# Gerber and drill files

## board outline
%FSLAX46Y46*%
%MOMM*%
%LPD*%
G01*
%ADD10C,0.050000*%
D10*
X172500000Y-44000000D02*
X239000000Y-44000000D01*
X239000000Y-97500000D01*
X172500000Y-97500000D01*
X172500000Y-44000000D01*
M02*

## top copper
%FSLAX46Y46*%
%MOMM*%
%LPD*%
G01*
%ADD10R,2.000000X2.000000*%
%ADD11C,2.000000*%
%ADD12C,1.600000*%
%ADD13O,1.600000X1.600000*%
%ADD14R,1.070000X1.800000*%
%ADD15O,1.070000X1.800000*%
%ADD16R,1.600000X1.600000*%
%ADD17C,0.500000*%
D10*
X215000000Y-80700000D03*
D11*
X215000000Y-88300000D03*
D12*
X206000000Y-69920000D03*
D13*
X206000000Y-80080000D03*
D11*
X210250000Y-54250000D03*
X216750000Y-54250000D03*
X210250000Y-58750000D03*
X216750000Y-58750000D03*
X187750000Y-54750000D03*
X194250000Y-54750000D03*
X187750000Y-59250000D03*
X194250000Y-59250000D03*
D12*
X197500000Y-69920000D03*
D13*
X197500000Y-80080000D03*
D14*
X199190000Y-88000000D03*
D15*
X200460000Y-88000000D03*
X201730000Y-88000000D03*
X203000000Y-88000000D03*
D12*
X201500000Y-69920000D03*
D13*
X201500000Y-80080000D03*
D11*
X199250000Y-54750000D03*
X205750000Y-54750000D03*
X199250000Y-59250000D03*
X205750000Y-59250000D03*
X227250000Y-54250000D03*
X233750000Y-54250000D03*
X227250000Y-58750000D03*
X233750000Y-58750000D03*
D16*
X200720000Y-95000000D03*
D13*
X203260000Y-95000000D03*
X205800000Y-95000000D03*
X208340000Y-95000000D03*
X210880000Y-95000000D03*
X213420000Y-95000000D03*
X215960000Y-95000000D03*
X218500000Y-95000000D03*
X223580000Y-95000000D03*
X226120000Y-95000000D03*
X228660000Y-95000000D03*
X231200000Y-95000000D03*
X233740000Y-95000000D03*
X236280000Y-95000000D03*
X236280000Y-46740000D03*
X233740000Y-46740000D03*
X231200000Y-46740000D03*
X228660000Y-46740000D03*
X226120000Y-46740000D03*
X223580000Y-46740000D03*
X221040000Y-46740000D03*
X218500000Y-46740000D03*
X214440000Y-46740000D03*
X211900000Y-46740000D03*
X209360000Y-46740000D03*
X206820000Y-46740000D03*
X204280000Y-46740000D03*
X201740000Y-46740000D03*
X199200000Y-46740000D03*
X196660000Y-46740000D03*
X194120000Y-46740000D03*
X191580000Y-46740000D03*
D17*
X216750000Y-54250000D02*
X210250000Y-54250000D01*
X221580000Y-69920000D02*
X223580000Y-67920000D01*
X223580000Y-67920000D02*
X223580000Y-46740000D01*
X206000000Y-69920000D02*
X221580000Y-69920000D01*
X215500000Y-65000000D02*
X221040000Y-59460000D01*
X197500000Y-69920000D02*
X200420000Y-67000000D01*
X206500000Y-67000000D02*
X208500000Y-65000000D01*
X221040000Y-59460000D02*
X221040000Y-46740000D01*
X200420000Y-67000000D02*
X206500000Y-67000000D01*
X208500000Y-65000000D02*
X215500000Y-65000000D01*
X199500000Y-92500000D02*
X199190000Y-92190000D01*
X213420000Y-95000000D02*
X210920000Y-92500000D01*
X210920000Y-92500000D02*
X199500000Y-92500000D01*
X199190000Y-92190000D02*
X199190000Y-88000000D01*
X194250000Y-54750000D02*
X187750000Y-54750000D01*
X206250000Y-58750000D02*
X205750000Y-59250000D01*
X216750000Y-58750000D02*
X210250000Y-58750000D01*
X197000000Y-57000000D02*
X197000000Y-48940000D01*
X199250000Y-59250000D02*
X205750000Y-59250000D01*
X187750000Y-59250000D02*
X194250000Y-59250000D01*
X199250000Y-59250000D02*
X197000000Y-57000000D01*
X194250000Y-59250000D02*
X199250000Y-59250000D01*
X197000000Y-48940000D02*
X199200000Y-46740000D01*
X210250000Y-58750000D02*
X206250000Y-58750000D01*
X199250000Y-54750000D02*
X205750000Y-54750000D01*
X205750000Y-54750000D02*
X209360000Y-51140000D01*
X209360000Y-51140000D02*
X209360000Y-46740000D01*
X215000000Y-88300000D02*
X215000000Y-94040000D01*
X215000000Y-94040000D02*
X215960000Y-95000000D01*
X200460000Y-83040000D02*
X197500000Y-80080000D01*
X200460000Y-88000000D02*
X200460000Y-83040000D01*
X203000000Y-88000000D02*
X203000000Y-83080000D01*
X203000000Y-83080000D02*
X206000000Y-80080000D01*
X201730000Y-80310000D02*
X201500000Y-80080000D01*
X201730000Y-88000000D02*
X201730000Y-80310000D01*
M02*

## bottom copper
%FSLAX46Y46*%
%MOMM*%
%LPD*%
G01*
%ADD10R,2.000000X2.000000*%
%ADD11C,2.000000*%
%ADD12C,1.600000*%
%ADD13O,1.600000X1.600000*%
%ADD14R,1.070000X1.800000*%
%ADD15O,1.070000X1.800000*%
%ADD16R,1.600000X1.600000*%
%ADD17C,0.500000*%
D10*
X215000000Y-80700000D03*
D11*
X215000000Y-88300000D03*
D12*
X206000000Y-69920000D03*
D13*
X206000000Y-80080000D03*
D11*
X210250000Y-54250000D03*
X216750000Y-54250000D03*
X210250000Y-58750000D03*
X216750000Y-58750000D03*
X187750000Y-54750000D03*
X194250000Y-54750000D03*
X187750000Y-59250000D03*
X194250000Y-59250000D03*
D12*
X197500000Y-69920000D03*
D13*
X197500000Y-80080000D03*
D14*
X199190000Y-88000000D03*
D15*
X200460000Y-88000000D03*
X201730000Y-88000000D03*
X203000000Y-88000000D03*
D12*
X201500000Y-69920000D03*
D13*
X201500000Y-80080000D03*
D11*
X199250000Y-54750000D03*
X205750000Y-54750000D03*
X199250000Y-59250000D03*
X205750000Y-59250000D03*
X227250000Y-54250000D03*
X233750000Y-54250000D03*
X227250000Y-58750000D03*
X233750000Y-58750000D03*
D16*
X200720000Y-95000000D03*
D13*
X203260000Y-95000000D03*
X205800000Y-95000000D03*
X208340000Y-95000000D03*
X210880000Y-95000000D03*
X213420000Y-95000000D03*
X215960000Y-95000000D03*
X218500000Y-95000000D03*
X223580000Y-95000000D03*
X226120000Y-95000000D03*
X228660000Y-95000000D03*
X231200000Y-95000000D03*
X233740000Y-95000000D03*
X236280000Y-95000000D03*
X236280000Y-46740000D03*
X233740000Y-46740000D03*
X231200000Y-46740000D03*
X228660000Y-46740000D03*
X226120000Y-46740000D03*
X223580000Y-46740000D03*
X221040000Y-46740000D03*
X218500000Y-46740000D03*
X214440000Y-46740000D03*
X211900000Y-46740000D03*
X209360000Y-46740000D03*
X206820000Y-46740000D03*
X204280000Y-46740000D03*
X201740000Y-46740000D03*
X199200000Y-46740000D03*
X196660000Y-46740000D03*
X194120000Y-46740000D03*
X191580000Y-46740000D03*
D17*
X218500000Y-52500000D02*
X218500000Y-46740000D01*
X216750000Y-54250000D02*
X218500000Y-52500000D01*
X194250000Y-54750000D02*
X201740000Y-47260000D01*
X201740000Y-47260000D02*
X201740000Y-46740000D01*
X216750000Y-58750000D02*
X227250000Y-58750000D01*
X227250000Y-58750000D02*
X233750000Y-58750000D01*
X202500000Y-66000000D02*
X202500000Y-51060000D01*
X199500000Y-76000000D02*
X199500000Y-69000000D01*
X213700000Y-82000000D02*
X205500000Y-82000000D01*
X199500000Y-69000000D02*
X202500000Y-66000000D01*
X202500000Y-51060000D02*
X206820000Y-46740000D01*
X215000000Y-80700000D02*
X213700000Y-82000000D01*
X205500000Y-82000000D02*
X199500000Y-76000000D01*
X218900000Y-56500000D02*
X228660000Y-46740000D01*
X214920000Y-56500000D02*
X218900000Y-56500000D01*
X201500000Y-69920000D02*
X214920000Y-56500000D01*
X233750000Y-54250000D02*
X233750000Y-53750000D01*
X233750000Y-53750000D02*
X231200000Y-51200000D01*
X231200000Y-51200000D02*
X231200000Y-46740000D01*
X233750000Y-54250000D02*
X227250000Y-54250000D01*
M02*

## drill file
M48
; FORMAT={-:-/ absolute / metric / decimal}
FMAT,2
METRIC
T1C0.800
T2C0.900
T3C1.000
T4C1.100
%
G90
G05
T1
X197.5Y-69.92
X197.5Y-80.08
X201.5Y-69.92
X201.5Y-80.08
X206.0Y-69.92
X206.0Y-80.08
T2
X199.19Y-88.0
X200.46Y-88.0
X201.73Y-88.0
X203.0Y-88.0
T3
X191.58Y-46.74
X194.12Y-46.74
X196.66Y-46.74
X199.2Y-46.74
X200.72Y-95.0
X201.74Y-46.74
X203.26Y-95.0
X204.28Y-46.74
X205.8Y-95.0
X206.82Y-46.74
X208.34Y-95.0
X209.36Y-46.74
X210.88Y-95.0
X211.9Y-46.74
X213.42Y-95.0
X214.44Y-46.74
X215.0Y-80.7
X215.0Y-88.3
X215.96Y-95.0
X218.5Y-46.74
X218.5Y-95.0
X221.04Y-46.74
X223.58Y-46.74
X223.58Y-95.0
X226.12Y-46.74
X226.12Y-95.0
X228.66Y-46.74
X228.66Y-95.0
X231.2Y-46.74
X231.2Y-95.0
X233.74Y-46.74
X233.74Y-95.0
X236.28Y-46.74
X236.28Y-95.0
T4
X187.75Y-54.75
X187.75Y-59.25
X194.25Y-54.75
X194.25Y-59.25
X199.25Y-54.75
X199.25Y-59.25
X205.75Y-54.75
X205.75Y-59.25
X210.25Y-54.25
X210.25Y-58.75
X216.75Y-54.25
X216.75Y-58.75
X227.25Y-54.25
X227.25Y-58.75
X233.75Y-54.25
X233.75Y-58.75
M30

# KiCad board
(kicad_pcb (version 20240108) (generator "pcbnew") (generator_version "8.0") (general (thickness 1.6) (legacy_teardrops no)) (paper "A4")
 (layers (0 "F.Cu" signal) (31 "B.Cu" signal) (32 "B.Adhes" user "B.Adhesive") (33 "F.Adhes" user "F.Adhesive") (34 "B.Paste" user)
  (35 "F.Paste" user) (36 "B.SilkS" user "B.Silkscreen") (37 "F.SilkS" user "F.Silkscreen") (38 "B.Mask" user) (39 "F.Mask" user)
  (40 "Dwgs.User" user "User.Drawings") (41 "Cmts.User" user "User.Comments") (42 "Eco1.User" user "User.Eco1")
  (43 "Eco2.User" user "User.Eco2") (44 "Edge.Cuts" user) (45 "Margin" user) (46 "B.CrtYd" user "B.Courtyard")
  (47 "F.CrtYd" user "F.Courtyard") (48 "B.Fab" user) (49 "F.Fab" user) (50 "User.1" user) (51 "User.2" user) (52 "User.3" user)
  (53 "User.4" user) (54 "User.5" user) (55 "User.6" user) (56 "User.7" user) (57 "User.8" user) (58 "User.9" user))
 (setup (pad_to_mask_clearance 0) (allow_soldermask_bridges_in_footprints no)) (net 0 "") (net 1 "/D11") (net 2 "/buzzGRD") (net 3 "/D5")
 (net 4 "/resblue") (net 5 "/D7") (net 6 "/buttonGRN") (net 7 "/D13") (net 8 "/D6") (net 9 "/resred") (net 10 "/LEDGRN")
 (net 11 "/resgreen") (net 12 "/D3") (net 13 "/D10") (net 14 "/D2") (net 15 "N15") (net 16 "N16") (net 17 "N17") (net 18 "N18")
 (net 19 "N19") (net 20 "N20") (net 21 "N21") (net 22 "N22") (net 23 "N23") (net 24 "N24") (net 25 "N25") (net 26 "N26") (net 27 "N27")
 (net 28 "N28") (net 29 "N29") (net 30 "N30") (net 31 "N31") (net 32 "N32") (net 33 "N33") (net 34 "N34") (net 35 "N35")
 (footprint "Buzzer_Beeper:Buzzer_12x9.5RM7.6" (layer "F.Cu") (at 215 80.7 -90)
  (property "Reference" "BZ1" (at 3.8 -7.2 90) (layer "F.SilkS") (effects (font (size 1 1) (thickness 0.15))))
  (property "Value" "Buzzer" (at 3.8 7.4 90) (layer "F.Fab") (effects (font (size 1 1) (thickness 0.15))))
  (pad "1" thru_hole rect (at 0 0 270) (size 2 2) (drill 1) (layers "*.Cu" "*.Mask") (remove_unused_layers no) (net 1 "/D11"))
  (pad "2" thru_hole circle (at 7.6 0 270) (size 2 2) (drill 1) (layers "*.Cu" "*.Mask") (remove_unused_layers no) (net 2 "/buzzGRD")))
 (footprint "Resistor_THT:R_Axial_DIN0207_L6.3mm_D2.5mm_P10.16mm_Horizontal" (layer "F.Cu") (at 206 69.92 -90)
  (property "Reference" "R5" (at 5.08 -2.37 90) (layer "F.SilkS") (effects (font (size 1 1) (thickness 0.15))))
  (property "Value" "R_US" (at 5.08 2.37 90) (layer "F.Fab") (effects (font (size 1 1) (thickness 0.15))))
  (pad "1" thru_hole circle (at 0 0 270) (size 1.6 1.6) (drill 0.8) (layers "*.Cu" "*.Mask") (remove_unused_layers no) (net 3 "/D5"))
  (pad "2" thru_hole oval (at 10.16 0 270) (size 1.6 1.6) (drill 0.8) (layers "*.Cu" "*.Mask") (remove_unused_layers no) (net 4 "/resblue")))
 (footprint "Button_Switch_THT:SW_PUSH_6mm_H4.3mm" (layer "F.Cu") (at 210.25 54.25)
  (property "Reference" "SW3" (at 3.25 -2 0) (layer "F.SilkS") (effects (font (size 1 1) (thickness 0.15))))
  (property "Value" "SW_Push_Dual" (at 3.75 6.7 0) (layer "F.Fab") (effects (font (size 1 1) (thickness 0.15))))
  (pad "1" thru_hole circle (at 0 0 90) (size 2 2) (drill 1.1) (layers "*.Cu" "*.Mask") (remove_unused_layers no) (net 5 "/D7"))
  (pad "1" thru_hole circle (at 6.5 0 90) (size 2 2) (drill 1.1) (layers "*.Cu" "*.Mask") (remove_unused_layers no) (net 5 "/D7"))
  (pad "2" thru_hole circle (at 0 4.5 90) (size 2 2) (drill 1.1) (layers "*.Cu" "*.Mask") (remove_unused_layers no) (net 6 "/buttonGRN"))
  (pad "2" thru_hole circle (at 6.5 4.5 90) (size 2 2) (drill 1.1) (layers "*.Cu" "*.Mask") (remove_unused_layers no) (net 6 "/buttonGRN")))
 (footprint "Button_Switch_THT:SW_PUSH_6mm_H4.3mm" (layer "F.Cu") (at 187.75 54.75)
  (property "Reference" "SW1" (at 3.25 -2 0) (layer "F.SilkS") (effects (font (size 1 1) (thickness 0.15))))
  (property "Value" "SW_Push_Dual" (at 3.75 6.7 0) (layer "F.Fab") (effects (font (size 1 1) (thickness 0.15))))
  (pad "1" thru_hole circle (at 0 0 90) (size 2 2) (drill 1.1) (layers "*.Cu" "*.Mask") (remove_unused_layers no) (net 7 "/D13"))
  (pad "1" thru_hole circle (at 6.5 0 90) (size 2 2) (drill 1.1) (layers "*.Cu" "*.Mask") (remove_unused_layers no) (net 7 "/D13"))
  (pad "2" thru_hole circle (at 0 4.5 90) (size 2 2) (drill 1.1) (layers "*.Cu" "*.Mask") (remove_unused_layers no) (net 6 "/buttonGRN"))
  (pad "2" thru_hole circle (at 6.5 4.5 90) (size 2 2) (drill 1.1) (layers "*.Cu" "*.Mask") (remove_unused_layers no) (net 6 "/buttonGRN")))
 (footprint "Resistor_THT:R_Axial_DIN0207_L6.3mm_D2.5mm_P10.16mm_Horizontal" (layer "F.Cu") (at 197.5 69.92 -90)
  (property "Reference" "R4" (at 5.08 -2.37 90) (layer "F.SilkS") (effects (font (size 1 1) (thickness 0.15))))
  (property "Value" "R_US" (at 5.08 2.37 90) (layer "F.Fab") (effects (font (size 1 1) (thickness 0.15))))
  (pad "1" thru_hole circle (at 0 0 270) (size 1.6 1.6) (drill 0.8) (layers "*.Cu" "*.Mask") (remove_unused_layers no) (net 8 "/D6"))
  (pad "2" thru_hole oval (at 10.16 0 270) (size 1.6 1.6) (drill 0.8) (layers "*.Cu" "*.Mask") (remove_unused_layers no) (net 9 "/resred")))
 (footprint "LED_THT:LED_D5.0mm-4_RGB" (layer "F.Cu") (at 199.19 88)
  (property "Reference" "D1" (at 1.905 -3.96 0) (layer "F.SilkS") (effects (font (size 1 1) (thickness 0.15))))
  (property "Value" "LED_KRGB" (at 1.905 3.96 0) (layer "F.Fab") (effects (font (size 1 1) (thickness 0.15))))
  (pad "1" thru_hole rect (at 0 0) (size 1.07 1.8) (drill 0.9) (layers "*.Cu" "*.Mask") (remove_unused_layers no) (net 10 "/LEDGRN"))
  (pad "2" thru_hole oval (at 1.27 0) (size 1.07 1.8) (drill 0.9) (layers "*.Cu" "*.Mask") (remove_unused_layers no) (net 9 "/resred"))
  (pad "3" thru_hole oval (at 2.54 0) (size 1.07 1.8) (drill 0.9) (layers "*.Cu" "*.Mask") (remove_unused_layers no) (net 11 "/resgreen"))
  (pad "4" thru_hole oval (at 3.81 0) (size 1.07 1.8) (drill 0.9) (layers "*.Cu" "*.Mask") (remove_unused_layers no) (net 4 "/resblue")))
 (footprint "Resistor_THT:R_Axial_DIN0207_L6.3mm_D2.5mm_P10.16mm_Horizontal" (layer "F.Cu") (at 201.5 69.92 -90)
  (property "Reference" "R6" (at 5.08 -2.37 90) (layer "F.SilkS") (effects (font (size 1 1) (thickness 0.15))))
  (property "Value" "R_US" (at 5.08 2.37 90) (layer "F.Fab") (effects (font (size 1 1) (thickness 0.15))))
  (pad "1" thru_hole circle (at 0 0 270) (size 1.6 1.6) (drill 0.8) (layers "*.Cu" "*.Mask") (remove_unused_layers no) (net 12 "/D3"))
  (pad "2" thru_hole oval (at 10.16 0 270) (size 1.6 1.6) (drill 0.8) (layers "*.Cu" "*.Mask") (remove_unused_layers no)
   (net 11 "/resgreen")))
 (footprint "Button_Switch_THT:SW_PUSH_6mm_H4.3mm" (layer "F.Cu") (at 199.25 54.75)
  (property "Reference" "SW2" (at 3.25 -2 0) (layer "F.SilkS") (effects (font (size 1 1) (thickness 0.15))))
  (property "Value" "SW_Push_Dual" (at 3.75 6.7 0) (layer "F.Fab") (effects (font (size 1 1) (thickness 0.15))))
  (pad "1" thru_hole circle (at 0 0 90) (size 2 2) (drill 1.1) (layers "*.Cu" "*.Mask") (remove_unused_layers no) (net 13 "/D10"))
  (pad "1" thru_hole circle (at 6.5 0 90) (size 2 2) (drill 1.1) (layers "*.Cu" "*.Mask") (remove_unused_layers no) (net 13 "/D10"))
  (pad "2" thru_hole circle (at 0 4.5 90) (size 2 2) (drill 1.1) (layers "*.Cu" "*.Mask") (remove_unused_layers no) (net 6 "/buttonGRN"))
  (pad "2" thru_hole circle (at 6.5 4.5 90) (size 2 2) (drill 1.1) (layers "*.Cu" "*.Mask") (remove_unused_layers no) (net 6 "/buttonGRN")))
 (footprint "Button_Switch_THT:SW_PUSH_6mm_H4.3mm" (layer "F.Cu") (at 227.25 54.25)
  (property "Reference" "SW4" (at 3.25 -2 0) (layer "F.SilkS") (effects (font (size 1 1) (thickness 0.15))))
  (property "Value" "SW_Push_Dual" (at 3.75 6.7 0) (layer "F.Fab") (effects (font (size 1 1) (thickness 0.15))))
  (pad "1" thru_hole circle (at 0 0 90) (size 2 2) (drill 1.1) (layers "*.Cu" "*.Mask") (remove_unused_layers no) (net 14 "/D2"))
  (pad "1" thru_hole circle (at 6.5 0 90) (size 2 2) (drill 1.1) (layers "*.Cu" "*.Mask") (remove_unused_layers no) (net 14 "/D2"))
  (pad "2" thru_hole circle (at 0 4.5 90) (size 2 2) (drill 1.1) (layers "*.Cu" "*.Mask") (remove_unused_layers no) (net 6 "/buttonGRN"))
  (pad "2" thru_hole circle (at 6.5 4.5 90) (size 2 2) (drill 1.1) (layers "*.Cu" "*.Mask") (remove_unused_layers no) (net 6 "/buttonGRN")))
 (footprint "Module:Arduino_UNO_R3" (layer "B.Cu") (at 200.72 95)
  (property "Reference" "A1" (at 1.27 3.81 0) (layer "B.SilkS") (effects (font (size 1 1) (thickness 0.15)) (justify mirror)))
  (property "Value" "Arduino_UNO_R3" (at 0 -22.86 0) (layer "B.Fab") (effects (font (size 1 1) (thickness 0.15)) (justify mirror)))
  (pad "1" thru_hole rect (at 0 0 270) (size 1.6 1.6) (drill 1) (layers "*.Cu" "*.Mask") (remove_unused_layers no) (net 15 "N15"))
  (pad "2" thru_hole oval (at 2.54 0 270) (size 1.6 1.6) (drill 1) (layers "*.Cu" "*.Mask") (remove_unused_layers no) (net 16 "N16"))
  (pad "3" thru_hole oval (at 5.08 0 270) (size 1.6 1.6) (drill 1) (layers "*.Cu" "*.Mask") (remove_unused_layers no) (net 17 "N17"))
  (pad "4" thru_hole oval (at 7.62 0 270) (size 1.6 1.6) (drill 1) (layers "*.Cu" "*.Mask") (remove_unused_layers no) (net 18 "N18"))
  (pad "5" thru_hole oval (at 10.16 0 270) (size 1.6 1.6) (drill 1) (layers "*.Cu" "*.Mask") (remove_unused_layers no) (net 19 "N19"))
  (pad "6" thru_hole oval (at 12.7 0 270) (size 1.6 1.6) (drill 1) (layers "*.Cu" "*.Mask") (remove_unused_layers no) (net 10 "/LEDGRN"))
  (pad "7" thru_hole oval (at 15.24 0 270) (size 1.6 1.6) (drill 1) (layers "*.Cu" "*.Mask") (remove_unused_layers no) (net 2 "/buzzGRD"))
  (pad "8" thru_hole oval (at 17.78 0 270) (size 1.6 1.6) (drill 1) (layers "*.Cu" "*.Mask") (remove_unused_layers no) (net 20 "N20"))
  (pad "9" thru_hole oval (at 22.86 0 270) (size 1.6 1.6) (drill 1) (layers "*.Cu" "*.Mask") (remove_unused_layers no) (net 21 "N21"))
  (pad "10" thru_hole oval (at 25.4 0 270) (size 1.6 1.6) (drill 1) (layers "*.Cu" "*.Mask") (remove_unused_layers no) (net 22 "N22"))
  (pad "11" thru_hole oval (at 27.94 0 270) (size 1.6 1.6) (drill 1) (layers "*.Cu" "*.Mask") (remove_unused_layers no) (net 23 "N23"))
  (pad "12" thru_hole oval (at 30.48 0 270) (size 1.6 1.6) (drill 1) (layers "*.Cu" "*.Mask") (remove_unused_layers no) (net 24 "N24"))
  (pad "13" thru_hole oval (at 33.02 0 270) (size 1.6 1.6) (drill 1) (layers "*.Cu" "*.Mask") (remove_unused_layers no) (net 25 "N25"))
  (pad "14" thru_hole oval (at 35.56 0 270) (size 1.6 1.6) (drill 1) (layers "*.Cu" "*.Mask") (remove_unused_layers no) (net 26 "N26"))
  (pad "15" thru_hole oval (at 35.56 -48.26 270) (size 1.6 1.6) (drill 1) (layers "*.Cu" "*.Mask") (remove_unused_layers no) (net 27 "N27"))
  (pad "16" thru_hole oval (at 33.02 -48.26 270) (size 1.6 1.6) (drill 1) (layers "*.Cu" "*.Mask") (remove_unused_layers no) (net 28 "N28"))
  (pad "17" thru_hole oval (at 30.48 -48.26 270) (size 1.6 1.6) (drill 1) (layers "*.Cu" "*.Mask") (remove_unused_layers no) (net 14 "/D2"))
  (pad "18" thru_hole oval (at 27.94 -48.26 270) (size 1.6 1.6) (drill 1) (layers "*.Cu" "*.Mask") (remove_unused_layers no) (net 12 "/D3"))
  (pad "19" thru_hole oval (at 25.4 -48.26 270) (size 1.6 1.6) (drill 1) (layers "*.Cu" "*.Mask") (remove_unused_layers no) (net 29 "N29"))
  (pad "20" thru_hole oval (at 22.86 -48.26 270) (size 1.6 1.6) (drill 1) (layers "*.Cu" "*.Mask") (remove_unused_layers no) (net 3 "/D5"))
  (pad "21" thru_hole oval (at 20.32 -48.26 270) (size 1.6 1.6) (drill 1) (layers "*.Cu" "*.Mask") (remove_unused_layers no) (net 8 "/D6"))
  (pad "22" thru_hole oval (at 17.78 -48.26 270) (size 1.6 1.6) (drill 1) (layers "*.Cu" "*.Mask") (remove_unused_layers no) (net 5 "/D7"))
  (pad "23" thru_hole oval (at 13.72 -48.26 270) (size 1.6 1.6) (drill 1) (layers "*.Cu" "*.Mask") (remove_unused_layers no) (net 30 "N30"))
  (pad "24" thru_hole oval (at 11.18 -48.26 270) (size 1.6 1.6) (drill 1) (layers "*.Cu" "*.Mask") (remove_unused_layers no) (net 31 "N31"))
  (pad "25" thru_hole oval (at 8.64 -48.26 270) (size 1.6 1.6) (drill 1) (layers "*.Cu" "*.Mask") (remove_unused_layers no) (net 13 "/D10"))
  (pad "26" thru_hole oval (at 6.1 -48.26 270) (size 1.6 1.6) (drill 1) (layers "*.Cu" "*.Mask") (remove_unused_layers no) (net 1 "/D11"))
  (pad "27" thru_hole oval (at 3.56 -48.26 270) (size 1.6 1.6) (drill 1) (layers "*.Cu" "*.Mask") (remove_unused_layers no) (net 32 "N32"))
  (pad "28" thru_hole oval (at 1.02 -48.26 270) (size 1.6 1.6) (drill 1) (layers "*.Cu" "*.Mask") (remove_unused_layers no) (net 7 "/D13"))
  (pad "29" thru_hole oval (at -1.52 -48.26 270) (size 1.6 1.6) (drill 1) (layers "*.Cu" "*.Mask") (remove_unused_layers no)
   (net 6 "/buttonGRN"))
  (pad "30" thru_hole oval (at -4.06 -48.26 270) (size 1.6 1.6) (drill 1) (layers "*.Cu" "*.Mask") (remove_unused_layers no) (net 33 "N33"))
  (pad "31" thru_hole oval (at -6.6 -48.26 270) (size 1.6 1.6) (drill 1) (layers "*.Cu" "*.Mask") (remove_unused_layers no) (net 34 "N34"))
  (pad "32" thru_hole oval (at -9.14 -48.26 270) (size 1.6 1.6) (drill 1) (layers "*.Cu" "*.Mask") (remove_unused_layers no) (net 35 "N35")))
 (gr_rect (start 172.5 44) (end 239 97.5) (stroke (width 0.05) (type default)) (fill none) (layer "Edge.Cuts"))
 (segment (start 216.75 54.25) (end 210.25 54.25) (width 0.5) (layer "F.Cu") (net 5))
 (segment (start 218.5 52.5) (end 218.5 46.74) (width 0.5) (layer "B.Cu") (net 5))
 (segment (start 216.75 54.25) (end 218.5 52.5) (width 0.5) (layer "B.Cu") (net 5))
 (segment (start 221.58 69.92) (end 223.58 67.92) (width 0.5) (layer "F.Cu") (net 3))
 (segment (start 223.58 67.92) (end 223.58 46.74) (width 0.5) (layer "F.Cu") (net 3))
 (segment (start 206 69.92) (end 221.58 69.92) (width 0.5) (layer "F.Cu") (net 3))
 (segment (start 215.5 65) (end 221.04 59.46) (width 0.5) (layer "F.Cu") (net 8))
 (segment (start 197.5 69.92) (end 200.42 67) (width 0.5) (layer "F.Cu") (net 8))
 (segment (start 206.5 67) (end 208.5 65) (width 0.5) (layer "F.Cu") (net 8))
 (segment (start 221.04 59.46) (end 221.04 46.74) (width 0.5) (layer "F.Cu") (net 8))
 (segment (start 200.42 67) (end 206.5 67) (width 0.5) (layer "F.Cu") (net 8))
 (segment (start 208.5 65) (end 215.5 65) (width 0.5) (layer "F.Cu") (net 8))
 (segment (start 199.5 92.5) (end 199.19 92.19) (width 0.5) (layer "F.Cu") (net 10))
 (segment (start 213.42 95) (end 210.92 92.5) (width 0.5) (layer "F.Cu") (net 10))
 (segment (start 210.92 92.5) (end 199.5 92.5) (width 0.5) (layer "F.Cu") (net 10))
 (segment (start 199.19 92.19) (end 199.19 88) (width 0.5) (layer "F.Cu") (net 10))
 (segment (start 194.25 54.75) (end 187.75 54.75) (width 0.5) (layer "F.Cu") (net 7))
 (segment (start 194.25 54.75) (end 201.74 47.26) (width 0.5) (layer "B.Cu") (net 7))
 (segment (start 201.74 47.26) (end 201.74 46.74) (width 0.5) (layer "B.Cu") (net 7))
 (segment (start 206.25 58.75) (end 205.75 59.25) (width 0.5) (layer "F.Cu") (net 6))
 (segment (start 216.75 58.75) (end 210.25 58.75) (width 0.5) (layer "F.Cu") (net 6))
 (segment (start 197 57) (end 197 48.94) (width 0.5) (layer "F.Cu") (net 6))
 (segment (start 199.25 59.25) (end 205.75 59.25) (width 0.5) (layer "F.Cu") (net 6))
 (segment (start 187.75 59.25) (end 194.25 59.25) (width 0.5) (layer "F.Cu") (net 6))
 (segment (start 199.25 59.25) (end 197 57) (width 0.5) (layer "F.Cu") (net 6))
 (segment (start 194.25 59.25) (end 199.25 59.25) (width 0.5) (layer "F.Cu") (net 6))
 (segment (start 197 48.94) (end 199.2 46.74) (width 0.5) (layer "F.Cu") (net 6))
 (segment (start 210.25 58.75) (end 206.25 58.75) (width 0.5) (layer "F.Cu") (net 6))
 (segment (start 216.75 58.75) (end 227.25 58.75) (width 0.5) (layer "B.Cu") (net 6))
 (segment (start 227.25 58.75) (end 233.75 58.75) (width 0.5) (layer "B.Cu") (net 6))
 (segment (start 202.5 66) (end 202.5 51.06) (width 0.5) (layer "B.Cu") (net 1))
 (segment (start 199.5 76) (end 199.5 69) (width 0.5) (layer "B.Cu") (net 1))
 (segment (start 213.7 82) (end 205.5 82) (width 0.5) (layer "B.Cu") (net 1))
 (segment (start 199.5 69) (end 202.5 66) (width 0.5) (layer "B.Cu") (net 1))
 (segment (start 202.5 51.06) (end 206.82 46.74) (width 0.5) (layer "B.Cu") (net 1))
 (segment (start 215 80.7) (end 213.7 82) (width 0.5) (layer "B.Cu") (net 1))
 (segment (start 205.5 82) (end 199.5 76) (width 0.5) (layer "B.Cu") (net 1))
 (segment (start 218.9 56.5) (end 228.66 46.74) (width 0.5) (layer "B.Cu") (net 12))
 (segment (start 214.92 56.5) (end 218.9 56.5) (width 0.5) (layer "B.Cu") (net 12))
 (segment (start 201.5 69.92) (end 214.92 56.5) (width 0.5) (layer "B.Cu") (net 12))
 (segment (start 199.25 54.75) (end 205.75 54.75) (width 0.5) (layer "F.Cu") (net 13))
 (segment (start 205.75 54.75) (end 209.36 51.14) (width 0.5) (layer "F.Cu") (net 13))
 (segment (start 209.36 51.14) (end 209.36 46.74) (width 0.5) (layer "F.Cu") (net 13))
 (segment (start 215 88.3) (end 215 94.04) (width 0.5) (layer "F.Cu") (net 2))
 (segment (start 215 94.04) (end 215.96 95) (width 0.5) (layer "F.Cu") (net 2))
 (segment (start 200.46 83.04) (end 197.5 80.08) (width 0.5) (layer "F.Cu") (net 9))
 (segment (start 200.46 88) (end 200.46 83.04) (width 0.5) (layer "F.Cu") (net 9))
 (segment (start 203 88) (end 203 83.08) (width 0.5) (layer "F.Cu") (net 4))
 (segment (start 203 83.08) (end 206 80.08) (width 0.5) (layer "F.Cu") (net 4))
 (segment (start 201.73 80.31) (end 201.5 80.08) (width 0.5) (layer "F.Cu") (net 11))
 (segment (start 201.73 88) (end 201.73 80.31) (width 0.5) (layer "F.Cu") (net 11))
 (segment (start 233.75 54.25) (end 233.75 53.75) (width 0.5) (layer "B.Cu") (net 14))
 (segment (start 233.75 53.75) (end 231.2 51.2) (width 0.5) (layer "B.Cu") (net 14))
 (segment (start 231.2 51.2) (end 231.2 46.74) (width 0.5) (layer "B.Cu") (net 14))
 (segment (start 233.75 54.25) (end 227.25 54.25) (width 0.5) (layer "B.Cu") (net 14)))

